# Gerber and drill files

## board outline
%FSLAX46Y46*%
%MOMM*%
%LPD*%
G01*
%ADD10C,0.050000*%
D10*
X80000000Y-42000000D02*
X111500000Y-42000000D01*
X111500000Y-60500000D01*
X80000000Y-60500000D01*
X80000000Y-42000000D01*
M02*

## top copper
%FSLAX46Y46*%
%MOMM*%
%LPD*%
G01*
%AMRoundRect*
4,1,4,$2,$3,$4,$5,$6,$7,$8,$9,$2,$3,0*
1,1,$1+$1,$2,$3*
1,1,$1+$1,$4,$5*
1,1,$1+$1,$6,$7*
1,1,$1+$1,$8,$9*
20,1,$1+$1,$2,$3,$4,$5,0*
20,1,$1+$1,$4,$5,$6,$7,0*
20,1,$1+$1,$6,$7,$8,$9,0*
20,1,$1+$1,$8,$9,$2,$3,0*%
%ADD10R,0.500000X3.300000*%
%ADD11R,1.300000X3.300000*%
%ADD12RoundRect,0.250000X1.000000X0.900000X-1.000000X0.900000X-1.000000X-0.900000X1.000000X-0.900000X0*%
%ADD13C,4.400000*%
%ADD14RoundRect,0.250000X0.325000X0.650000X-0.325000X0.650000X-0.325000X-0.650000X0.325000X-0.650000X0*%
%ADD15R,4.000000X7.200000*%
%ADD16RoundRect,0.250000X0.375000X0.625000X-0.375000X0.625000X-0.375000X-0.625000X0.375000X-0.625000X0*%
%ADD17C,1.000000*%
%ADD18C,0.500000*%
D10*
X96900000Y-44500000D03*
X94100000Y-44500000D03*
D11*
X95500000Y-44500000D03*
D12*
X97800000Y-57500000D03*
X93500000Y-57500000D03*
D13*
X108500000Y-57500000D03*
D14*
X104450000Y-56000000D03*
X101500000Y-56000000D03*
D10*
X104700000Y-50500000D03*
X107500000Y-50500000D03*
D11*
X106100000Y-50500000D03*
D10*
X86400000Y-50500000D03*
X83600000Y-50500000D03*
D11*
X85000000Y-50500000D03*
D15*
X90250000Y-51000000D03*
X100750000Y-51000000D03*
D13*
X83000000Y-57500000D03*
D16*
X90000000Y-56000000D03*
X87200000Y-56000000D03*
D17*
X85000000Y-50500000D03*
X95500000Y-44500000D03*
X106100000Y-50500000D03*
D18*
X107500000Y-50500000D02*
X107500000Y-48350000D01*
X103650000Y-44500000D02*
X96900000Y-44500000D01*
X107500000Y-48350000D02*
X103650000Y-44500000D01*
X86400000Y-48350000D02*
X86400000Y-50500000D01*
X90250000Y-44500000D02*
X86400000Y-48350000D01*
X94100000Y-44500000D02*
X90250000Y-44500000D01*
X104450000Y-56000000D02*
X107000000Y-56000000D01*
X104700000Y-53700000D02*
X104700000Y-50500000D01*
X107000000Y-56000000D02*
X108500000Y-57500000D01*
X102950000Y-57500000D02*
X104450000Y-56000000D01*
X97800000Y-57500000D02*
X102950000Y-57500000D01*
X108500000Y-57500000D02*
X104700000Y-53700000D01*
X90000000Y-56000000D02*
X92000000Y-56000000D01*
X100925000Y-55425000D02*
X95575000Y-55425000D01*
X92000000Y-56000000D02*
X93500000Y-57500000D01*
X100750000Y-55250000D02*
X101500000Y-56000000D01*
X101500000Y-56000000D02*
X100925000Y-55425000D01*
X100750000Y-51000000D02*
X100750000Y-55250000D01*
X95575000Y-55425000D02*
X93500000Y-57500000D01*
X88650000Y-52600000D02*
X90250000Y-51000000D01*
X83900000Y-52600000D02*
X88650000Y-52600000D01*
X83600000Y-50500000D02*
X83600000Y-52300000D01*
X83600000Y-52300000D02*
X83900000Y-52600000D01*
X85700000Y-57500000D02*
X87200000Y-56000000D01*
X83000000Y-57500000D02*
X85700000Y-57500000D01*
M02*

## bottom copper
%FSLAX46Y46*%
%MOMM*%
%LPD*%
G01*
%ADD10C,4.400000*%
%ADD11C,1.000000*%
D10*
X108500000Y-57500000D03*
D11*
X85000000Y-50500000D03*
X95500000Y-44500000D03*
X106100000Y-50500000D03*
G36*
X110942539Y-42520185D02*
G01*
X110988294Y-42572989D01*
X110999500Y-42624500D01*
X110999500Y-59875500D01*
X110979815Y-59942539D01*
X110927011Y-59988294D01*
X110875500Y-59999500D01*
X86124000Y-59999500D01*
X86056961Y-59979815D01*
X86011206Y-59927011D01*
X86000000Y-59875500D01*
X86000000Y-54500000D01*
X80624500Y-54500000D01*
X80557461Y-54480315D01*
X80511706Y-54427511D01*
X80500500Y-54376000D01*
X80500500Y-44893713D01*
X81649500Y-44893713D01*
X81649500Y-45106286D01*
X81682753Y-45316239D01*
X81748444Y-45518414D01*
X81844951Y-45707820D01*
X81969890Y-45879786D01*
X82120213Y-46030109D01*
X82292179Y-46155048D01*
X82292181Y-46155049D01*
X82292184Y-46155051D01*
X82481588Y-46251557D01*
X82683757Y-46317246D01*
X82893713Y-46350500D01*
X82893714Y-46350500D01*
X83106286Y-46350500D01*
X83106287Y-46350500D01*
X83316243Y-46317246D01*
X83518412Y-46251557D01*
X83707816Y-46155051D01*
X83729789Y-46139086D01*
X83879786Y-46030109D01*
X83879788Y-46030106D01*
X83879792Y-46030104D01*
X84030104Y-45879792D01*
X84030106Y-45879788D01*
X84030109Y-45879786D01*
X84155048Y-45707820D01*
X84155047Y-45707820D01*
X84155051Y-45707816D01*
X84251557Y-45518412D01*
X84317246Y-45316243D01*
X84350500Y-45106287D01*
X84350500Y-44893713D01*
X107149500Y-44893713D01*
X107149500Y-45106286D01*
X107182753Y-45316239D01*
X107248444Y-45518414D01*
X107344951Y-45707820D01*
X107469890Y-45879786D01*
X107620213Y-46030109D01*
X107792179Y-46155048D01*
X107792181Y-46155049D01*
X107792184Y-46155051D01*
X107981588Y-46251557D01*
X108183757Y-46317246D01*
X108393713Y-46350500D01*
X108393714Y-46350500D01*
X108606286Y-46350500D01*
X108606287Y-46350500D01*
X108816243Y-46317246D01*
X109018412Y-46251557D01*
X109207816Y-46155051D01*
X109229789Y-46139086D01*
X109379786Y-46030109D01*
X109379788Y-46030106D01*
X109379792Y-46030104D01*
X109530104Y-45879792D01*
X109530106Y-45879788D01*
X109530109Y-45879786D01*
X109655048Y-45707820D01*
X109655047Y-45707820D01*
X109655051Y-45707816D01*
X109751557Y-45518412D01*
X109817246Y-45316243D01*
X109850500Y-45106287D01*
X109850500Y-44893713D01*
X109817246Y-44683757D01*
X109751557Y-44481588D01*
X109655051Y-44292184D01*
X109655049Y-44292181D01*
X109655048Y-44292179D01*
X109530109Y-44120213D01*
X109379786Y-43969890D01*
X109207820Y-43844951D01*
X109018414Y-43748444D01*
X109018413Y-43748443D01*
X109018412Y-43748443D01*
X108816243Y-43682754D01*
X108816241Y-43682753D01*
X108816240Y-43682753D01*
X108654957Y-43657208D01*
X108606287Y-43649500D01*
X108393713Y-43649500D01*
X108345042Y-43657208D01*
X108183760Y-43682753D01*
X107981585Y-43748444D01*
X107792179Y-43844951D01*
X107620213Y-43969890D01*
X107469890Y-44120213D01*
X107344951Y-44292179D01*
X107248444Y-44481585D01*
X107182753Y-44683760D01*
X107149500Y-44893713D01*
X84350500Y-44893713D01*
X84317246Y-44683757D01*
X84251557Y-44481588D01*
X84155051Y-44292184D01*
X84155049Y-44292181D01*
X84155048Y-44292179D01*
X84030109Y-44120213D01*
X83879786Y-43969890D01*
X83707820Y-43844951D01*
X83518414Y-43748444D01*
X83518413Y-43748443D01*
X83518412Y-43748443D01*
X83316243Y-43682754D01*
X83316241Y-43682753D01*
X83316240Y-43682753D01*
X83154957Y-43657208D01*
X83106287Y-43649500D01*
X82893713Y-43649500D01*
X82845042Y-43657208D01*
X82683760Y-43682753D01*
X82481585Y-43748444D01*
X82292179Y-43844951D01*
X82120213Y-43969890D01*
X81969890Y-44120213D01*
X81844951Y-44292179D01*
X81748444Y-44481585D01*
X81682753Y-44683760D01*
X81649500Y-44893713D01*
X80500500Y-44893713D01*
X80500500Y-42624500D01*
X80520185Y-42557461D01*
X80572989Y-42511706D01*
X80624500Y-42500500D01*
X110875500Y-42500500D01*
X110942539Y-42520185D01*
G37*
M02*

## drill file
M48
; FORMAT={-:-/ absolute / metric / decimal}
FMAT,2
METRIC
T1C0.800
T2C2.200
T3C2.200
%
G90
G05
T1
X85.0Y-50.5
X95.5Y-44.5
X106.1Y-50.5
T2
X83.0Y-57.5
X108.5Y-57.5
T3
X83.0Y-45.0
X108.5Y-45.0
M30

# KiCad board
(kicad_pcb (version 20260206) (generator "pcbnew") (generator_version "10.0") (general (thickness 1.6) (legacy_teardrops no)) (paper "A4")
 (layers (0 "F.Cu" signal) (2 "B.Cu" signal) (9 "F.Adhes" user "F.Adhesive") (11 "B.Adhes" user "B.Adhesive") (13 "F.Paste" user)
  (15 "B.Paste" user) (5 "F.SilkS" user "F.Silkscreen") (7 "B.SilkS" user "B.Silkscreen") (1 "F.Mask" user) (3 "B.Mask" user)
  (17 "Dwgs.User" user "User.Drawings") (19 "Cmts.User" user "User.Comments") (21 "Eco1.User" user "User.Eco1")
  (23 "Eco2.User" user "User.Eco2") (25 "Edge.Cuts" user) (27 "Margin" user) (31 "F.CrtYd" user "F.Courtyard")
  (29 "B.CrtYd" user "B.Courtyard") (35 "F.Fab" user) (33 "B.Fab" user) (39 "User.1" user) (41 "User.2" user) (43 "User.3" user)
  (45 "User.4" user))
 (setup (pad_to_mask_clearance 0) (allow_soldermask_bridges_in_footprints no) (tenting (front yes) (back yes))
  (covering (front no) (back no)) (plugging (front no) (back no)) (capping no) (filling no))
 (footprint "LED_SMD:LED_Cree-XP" (layer "F.Cu") (at 95.5 44.5 180)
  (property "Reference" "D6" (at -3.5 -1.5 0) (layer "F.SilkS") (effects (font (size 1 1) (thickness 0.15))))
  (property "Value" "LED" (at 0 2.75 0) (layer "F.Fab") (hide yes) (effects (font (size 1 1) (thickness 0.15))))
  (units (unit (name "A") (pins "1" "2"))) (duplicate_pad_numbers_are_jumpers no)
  (pad "" smd rect (at 0 -1 180) (size 1.01 0.75) (layers "F.Paste"))
  (pad "" smd rect (at 0 0 180) (size 1.01 0.75) (layers "F.Paste"))
  (pad "" smd rect (at 0 1 180) (size 1.01 0.75) (layers "F.Paste"))
  (pad "1" smd rect (at -1.4 0 180) (size 0.5 3.3) (layers "F.Cu" "F.Mask" "F.Paste") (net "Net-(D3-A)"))
  (pad "2" smd rect (at 1.4 0 180) (size 0.5 3.3) (layers "F.Cu" "F.Mask" "F.Paste") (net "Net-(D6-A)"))
  (pad "3" smd rect (at 0 0 180) (size 1.3 3.3) (layers "F.Cu" "F.Mask") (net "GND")))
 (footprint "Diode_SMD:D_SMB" (layer "F.Cu") (at 95.65 57.5 180)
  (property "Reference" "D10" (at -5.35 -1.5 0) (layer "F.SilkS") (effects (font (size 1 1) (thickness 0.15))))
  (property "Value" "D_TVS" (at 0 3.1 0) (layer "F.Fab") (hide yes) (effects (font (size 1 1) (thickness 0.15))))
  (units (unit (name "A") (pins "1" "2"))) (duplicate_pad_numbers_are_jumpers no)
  (pad "1" smd roundrect (at -2.15 0 180) (size 2.5 2.3) (layers "F.Cu" "F.Mask" "F.Paste") (roundrect_rratio 0.1086956522) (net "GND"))
  (pad "2" smd roundrect (at 2.15 0 180) (size 2.5 2.3) (layers "F.Cu" "F.Mask" "F.Paste") (roundrect_rratio 0.1086956522)
   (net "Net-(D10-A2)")))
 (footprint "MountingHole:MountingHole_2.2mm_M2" (layer "F.Cu") (at 108.5 45)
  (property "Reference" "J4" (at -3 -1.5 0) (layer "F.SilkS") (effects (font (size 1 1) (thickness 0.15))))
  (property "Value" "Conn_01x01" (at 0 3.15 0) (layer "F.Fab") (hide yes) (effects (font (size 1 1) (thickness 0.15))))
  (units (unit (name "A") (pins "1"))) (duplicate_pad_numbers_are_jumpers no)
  (pad "" np_thru_hole circle (at 0 0) (size 2.2 2.2) (drill 2.2) (layers "*.Cu" "*.Mask")))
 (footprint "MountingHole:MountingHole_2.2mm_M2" (layer "F.Cu") (at 83 45)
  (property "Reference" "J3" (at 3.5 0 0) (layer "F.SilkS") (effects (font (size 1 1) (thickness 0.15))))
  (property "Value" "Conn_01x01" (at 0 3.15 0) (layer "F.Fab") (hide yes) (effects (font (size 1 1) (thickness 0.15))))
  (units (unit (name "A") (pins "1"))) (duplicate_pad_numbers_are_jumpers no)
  (pad "" np_thru_hole circle (at 0 0) (size 2.2 2.2) (drill 2.2) (layers "*.Cu" "*.Mask")))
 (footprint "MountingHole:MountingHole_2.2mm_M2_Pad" (layer "F.Cu") (at 108.5 57.5)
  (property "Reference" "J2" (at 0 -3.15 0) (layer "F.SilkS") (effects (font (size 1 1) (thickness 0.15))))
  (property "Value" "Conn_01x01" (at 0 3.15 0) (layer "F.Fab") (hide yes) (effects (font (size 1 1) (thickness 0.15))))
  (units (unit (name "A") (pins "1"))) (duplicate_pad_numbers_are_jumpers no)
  (pad "1" thru_hole circle (at 0 0) (size 4.4 4.4) (drill 2.2) (layers "*.Cu" "*.Mask") (remove_unused_layers no) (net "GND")
   (zone_connect 2)))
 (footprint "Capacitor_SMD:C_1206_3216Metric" (layer "F.Cu") (at 102.975 56 180)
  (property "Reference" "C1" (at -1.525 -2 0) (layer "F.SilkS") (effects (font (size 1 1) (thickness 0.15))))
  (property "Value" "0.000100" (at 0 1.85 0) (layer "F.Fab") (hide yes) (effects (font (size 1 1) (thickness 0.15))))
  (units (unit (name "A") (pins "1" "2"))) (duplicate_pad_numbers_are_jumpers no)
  (pad "1" smd roundrect (at -1.475 0 180) (size 1.15 1.8) (layers "F.Cu" "F.Mask" "F.Paste") (roundrect_rratio 0.217391) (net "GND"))
  (pad "2" smd roundrect (at 1.475 0 180) (size 1.15 1.8) (layers "F.Cu" "F.Mask" "F.Paste") (roundrect_rratio 0.217391)
   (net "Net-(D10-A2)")))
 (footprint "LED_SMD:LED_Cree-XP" (layer "F.Cu") (at 106.1 50.5)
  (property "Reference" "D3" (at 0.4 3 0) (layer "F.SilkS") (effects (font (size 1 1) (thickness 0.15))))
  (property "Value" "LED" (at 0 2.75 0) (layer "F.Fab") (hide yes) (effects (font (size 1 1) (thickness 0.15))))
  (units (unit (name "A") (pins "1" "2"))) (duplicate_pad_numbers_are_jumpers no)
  (pad "" smd rect (at 0 -1) (size 1.01 0.75) (layers "F.Paste"))
  (pad "" smd rect (at 0 0) (size 1.01 0.75) (layers "F.Paste"))
  (pad "" smd rect (at 0 1) (size 1.01 0.75) (layers "F.Paste"))
  (pad "1" smd rect (at -1.4 0) (size 0.5 3.3) (layers "F.Cu" "F.Mask" "F.Paste") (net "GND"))
  (pad "2" smd rect (at 1.4 0) (size 0.5 3.3) (layers "F.Cu" "F.Mask" "F.Paste") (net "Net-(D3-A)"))
  (pad "3" smd rect (at 0 0) (size 1.3 3.3) (layers "F.Cu" "F.Mask") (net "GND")))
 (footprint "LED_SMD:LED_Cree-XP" (layer "F.Cu") (at 85 50.5 180)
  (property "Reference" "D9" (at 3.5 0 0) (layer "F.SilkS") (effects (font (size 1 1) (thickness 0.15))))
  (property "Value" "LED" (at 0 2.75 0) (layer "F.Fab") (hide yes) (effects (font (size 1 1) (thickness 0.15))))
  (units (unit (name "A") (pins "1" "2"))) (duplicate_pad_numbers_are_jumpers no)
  (pad "" smd rect (at 0 -1 180) (size 1.01 0.75) (layers "F.Paste"))
  (pad "" smd rect (at 0 0 180) (size 1.01 0.75) (layers "F.Paste"))
  (pad "" smd rect (at 0 1 180) (size 1.01 0.75) (layers "F.Paste"))
  (pad "1" smd rect (at -1.4 0 180) (size 0.5 3.3) (layers "F.Cu" "F.Mask" "F.Paste") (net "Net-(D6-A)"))
  (pad "2" smd rect (at 1.4 0 180) (size 0.5 3.3) (layers "F.Cu" "F.Mask" "F.Paste") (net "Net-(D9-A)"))
  (pad "3" smd rect (at 0 0 180) (size 1.3 3.3) (layers "F.Cu" "F.Mask") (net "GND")))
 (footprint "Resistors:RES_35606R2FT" (layer "F.Cu") (at 95.5 51)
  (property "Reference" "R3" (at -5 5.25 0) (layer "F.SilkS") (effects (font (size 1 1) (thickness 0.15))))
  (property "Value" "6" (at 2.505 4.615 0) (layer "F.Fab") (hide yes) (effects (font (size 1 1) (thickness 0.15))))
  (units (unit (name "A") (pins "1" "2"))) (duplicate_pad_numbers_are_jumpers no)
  (pad "1" smd rect (at -5.25 0) (size 4 7.2) (layers "F.Cu" "F.Mask" "F.Paste") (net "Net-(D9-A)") (solder_mask_margin 0.102))
  (pad "2" smd rect (at 5.25 0) (size 4 7.2) (layers "F.Cu" "F.Mask" "F.Paste") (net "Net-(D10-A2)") (solder_mask_margin 0.102)))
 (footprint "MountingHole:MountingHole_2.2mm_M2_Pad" (layer "F.Cu") (at 83 57.5)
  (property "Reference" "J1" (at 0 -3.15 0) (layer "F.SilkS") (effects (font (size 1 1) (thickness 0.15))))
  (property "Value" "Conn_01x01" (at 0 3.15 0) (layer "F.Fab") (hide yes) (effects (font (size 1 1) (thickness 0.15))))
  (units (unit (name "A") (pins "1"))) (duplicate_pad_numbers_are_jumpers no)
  (pad "1" thru_hole circle (at 0 0) (size 4.4 4.4) (drill 2.2) (layers "*.Cu" "F.Mask") (remove_unused_layers yes) (keep_end_layers no)
   (zone_layer_connections) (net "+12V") (clearance 1) (zone_connect 2)))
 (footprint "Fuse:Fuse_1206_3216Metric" (layer "F.Cu") (at 88.6 56 180)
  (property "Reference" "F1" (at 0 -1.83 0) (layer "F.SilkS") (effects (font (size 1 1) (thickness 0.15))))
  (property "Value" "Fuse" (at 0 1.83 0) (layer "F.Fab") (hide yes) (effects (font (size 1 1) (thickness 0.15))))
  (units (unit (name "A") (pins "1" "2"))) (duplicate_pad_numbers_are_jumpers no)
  (pad "1" smd roundrect (at -1.4 0 180) (size 1.25 1.75) (layers "F.Cu" "F.Mask" "F.Paste") (roundrect_rratio 0.2) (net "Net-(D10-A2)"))
  (pad "2" smd roundrect (at 1.4 0 180) (size 1.25 1.75) (layers "F.Cu" "F.Mask" "F.Paste") (roundrect_rratio 0.2) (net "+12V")))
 (gr_rect (start 80 42) (end 111.5 60.5) (stroke (width 0.05) (type default)) (fill no) (layer "Edge.Cuts"))
 (segment (start 107.5 50.5) (end 107.5 48.35) (width 0.5) (layer "F.Cu") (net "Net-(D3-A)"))
 (segment (start 103.65 44.5) (end 96.9 44.5) (width 0.5) (layer "F.Cu") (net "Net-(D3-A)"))
 (segment (start 107.5 48.35) (end 103.65 44.5) (width 0.5) (layer "F.Cu") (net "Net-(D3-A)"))
 (segment (start 86.4 48.35) (end 86.4 50.5) (width 0.5) (layer "F.Cu") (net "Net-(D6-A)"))
 (segment (start 90.25 44.5) (end 86.4 48.35) (width 0.5) (layer "F.Cu") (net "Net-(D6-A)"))
 (segment (start 94.1 44.5) (end 90.25 44.5) (width 0.5) (layer "F.Cu") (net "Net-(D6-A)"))
 (segment (start 104.45 56) (end 107 56) (width 0.5) (layer "F.Cu") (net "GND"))
 (segment (start 104.7 53.7) (end 104.7 50.5) (width 0.5) (layer "F.Cu") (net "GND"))
 (segment (start 107 56) (end 108.5 57.5) (width 0.5) (layer "F.Cu") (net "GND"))
 (segment (start 102.95 57.5) (end 104.45 56) (width 0.5) (layer "F.Cu") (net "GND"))
 (segment (start 97.8 57.5) (end 102.95 57.5) (width 0.5) (layer "F.Cu") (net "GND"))
 (segment (start 108.5 57.5) (end 104.7 53.7) (width 0.5) (layer "F.Cu") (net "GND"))
 (via (at 85 50.5) (size 1) (drill 0.8) (layers "F.Cu" "B.Cu") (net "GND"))
 (via (at 95.5 44.5) (size 1) (drill 0.8) (layers "F.Cu" "B.Cu") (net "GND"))
 (via (at 106.1 50.5) (size 1) (drill 0.8) (layers "F.Cu" "B.Cu") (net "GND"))
 (segment (start 90 56) (end 92 56) (width 0.5) (layer "F.Cu") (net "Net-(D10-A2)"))
 (segment (start 100.925 55.425) (end 95.575 55.425) (width 0.5) (layer "F.Cu") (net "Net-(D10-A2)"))
 (segment (start 92 56) (end 93.5 57.5) (width 0.5) (layer "F.Cu") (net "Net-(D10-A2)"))
 (segment (start 100.75 55.25) (end 101.5 56) (width 0.5) (layer "F.Cu") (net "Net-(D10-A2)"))
 (segment (start 101.5 56) (end 100.925 55.425) (width 0.5) (layer "F.Cu") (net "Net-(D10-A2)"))
 (segment (start 100.75 51) (end 100.75 55.25) (width 0.5) (layer "F.Cu") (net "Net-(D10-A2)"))
 (segment (start 95.575 55.425) (end 93.5 57.5) (width 0.5) (layer "F.Cu") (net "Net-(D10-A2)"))
 (segment (start 88.65 52.6) (end 90.25 51) (width 0.5) (layer "F.Cu") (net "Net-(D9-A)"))
 (segment (start 83.9 52.6) (end 88.65 52.6) (width 0.5) (layer "F.Cu") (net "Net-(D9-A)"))
 (segment (start 83.6 50.5) (end 83.6 52.3) (width 0.5) (layer "F.Cu") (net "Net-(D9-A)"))
 (segment (start 83.6 52.3) (end 83.9 52.6) (width 0.5) (layer "F.Cu") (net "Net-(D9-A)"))
 (segment (start 85.7 57.5) (end 87.2 56) (width 0.5) (layer "F.Cu") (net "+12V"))
 (segment (start 83 57.5) (end 85.7 57.5) (width 0.5) (layer "F.Cu") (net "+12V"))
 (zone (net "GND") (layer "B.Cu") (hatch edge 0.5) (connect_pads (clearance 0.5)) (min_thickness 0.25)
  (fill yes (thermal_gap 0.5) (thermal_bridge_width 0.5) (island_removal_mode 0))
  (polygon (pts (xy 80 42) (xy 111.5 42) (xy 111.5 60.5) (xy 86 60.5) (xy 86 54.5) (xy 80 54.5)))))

